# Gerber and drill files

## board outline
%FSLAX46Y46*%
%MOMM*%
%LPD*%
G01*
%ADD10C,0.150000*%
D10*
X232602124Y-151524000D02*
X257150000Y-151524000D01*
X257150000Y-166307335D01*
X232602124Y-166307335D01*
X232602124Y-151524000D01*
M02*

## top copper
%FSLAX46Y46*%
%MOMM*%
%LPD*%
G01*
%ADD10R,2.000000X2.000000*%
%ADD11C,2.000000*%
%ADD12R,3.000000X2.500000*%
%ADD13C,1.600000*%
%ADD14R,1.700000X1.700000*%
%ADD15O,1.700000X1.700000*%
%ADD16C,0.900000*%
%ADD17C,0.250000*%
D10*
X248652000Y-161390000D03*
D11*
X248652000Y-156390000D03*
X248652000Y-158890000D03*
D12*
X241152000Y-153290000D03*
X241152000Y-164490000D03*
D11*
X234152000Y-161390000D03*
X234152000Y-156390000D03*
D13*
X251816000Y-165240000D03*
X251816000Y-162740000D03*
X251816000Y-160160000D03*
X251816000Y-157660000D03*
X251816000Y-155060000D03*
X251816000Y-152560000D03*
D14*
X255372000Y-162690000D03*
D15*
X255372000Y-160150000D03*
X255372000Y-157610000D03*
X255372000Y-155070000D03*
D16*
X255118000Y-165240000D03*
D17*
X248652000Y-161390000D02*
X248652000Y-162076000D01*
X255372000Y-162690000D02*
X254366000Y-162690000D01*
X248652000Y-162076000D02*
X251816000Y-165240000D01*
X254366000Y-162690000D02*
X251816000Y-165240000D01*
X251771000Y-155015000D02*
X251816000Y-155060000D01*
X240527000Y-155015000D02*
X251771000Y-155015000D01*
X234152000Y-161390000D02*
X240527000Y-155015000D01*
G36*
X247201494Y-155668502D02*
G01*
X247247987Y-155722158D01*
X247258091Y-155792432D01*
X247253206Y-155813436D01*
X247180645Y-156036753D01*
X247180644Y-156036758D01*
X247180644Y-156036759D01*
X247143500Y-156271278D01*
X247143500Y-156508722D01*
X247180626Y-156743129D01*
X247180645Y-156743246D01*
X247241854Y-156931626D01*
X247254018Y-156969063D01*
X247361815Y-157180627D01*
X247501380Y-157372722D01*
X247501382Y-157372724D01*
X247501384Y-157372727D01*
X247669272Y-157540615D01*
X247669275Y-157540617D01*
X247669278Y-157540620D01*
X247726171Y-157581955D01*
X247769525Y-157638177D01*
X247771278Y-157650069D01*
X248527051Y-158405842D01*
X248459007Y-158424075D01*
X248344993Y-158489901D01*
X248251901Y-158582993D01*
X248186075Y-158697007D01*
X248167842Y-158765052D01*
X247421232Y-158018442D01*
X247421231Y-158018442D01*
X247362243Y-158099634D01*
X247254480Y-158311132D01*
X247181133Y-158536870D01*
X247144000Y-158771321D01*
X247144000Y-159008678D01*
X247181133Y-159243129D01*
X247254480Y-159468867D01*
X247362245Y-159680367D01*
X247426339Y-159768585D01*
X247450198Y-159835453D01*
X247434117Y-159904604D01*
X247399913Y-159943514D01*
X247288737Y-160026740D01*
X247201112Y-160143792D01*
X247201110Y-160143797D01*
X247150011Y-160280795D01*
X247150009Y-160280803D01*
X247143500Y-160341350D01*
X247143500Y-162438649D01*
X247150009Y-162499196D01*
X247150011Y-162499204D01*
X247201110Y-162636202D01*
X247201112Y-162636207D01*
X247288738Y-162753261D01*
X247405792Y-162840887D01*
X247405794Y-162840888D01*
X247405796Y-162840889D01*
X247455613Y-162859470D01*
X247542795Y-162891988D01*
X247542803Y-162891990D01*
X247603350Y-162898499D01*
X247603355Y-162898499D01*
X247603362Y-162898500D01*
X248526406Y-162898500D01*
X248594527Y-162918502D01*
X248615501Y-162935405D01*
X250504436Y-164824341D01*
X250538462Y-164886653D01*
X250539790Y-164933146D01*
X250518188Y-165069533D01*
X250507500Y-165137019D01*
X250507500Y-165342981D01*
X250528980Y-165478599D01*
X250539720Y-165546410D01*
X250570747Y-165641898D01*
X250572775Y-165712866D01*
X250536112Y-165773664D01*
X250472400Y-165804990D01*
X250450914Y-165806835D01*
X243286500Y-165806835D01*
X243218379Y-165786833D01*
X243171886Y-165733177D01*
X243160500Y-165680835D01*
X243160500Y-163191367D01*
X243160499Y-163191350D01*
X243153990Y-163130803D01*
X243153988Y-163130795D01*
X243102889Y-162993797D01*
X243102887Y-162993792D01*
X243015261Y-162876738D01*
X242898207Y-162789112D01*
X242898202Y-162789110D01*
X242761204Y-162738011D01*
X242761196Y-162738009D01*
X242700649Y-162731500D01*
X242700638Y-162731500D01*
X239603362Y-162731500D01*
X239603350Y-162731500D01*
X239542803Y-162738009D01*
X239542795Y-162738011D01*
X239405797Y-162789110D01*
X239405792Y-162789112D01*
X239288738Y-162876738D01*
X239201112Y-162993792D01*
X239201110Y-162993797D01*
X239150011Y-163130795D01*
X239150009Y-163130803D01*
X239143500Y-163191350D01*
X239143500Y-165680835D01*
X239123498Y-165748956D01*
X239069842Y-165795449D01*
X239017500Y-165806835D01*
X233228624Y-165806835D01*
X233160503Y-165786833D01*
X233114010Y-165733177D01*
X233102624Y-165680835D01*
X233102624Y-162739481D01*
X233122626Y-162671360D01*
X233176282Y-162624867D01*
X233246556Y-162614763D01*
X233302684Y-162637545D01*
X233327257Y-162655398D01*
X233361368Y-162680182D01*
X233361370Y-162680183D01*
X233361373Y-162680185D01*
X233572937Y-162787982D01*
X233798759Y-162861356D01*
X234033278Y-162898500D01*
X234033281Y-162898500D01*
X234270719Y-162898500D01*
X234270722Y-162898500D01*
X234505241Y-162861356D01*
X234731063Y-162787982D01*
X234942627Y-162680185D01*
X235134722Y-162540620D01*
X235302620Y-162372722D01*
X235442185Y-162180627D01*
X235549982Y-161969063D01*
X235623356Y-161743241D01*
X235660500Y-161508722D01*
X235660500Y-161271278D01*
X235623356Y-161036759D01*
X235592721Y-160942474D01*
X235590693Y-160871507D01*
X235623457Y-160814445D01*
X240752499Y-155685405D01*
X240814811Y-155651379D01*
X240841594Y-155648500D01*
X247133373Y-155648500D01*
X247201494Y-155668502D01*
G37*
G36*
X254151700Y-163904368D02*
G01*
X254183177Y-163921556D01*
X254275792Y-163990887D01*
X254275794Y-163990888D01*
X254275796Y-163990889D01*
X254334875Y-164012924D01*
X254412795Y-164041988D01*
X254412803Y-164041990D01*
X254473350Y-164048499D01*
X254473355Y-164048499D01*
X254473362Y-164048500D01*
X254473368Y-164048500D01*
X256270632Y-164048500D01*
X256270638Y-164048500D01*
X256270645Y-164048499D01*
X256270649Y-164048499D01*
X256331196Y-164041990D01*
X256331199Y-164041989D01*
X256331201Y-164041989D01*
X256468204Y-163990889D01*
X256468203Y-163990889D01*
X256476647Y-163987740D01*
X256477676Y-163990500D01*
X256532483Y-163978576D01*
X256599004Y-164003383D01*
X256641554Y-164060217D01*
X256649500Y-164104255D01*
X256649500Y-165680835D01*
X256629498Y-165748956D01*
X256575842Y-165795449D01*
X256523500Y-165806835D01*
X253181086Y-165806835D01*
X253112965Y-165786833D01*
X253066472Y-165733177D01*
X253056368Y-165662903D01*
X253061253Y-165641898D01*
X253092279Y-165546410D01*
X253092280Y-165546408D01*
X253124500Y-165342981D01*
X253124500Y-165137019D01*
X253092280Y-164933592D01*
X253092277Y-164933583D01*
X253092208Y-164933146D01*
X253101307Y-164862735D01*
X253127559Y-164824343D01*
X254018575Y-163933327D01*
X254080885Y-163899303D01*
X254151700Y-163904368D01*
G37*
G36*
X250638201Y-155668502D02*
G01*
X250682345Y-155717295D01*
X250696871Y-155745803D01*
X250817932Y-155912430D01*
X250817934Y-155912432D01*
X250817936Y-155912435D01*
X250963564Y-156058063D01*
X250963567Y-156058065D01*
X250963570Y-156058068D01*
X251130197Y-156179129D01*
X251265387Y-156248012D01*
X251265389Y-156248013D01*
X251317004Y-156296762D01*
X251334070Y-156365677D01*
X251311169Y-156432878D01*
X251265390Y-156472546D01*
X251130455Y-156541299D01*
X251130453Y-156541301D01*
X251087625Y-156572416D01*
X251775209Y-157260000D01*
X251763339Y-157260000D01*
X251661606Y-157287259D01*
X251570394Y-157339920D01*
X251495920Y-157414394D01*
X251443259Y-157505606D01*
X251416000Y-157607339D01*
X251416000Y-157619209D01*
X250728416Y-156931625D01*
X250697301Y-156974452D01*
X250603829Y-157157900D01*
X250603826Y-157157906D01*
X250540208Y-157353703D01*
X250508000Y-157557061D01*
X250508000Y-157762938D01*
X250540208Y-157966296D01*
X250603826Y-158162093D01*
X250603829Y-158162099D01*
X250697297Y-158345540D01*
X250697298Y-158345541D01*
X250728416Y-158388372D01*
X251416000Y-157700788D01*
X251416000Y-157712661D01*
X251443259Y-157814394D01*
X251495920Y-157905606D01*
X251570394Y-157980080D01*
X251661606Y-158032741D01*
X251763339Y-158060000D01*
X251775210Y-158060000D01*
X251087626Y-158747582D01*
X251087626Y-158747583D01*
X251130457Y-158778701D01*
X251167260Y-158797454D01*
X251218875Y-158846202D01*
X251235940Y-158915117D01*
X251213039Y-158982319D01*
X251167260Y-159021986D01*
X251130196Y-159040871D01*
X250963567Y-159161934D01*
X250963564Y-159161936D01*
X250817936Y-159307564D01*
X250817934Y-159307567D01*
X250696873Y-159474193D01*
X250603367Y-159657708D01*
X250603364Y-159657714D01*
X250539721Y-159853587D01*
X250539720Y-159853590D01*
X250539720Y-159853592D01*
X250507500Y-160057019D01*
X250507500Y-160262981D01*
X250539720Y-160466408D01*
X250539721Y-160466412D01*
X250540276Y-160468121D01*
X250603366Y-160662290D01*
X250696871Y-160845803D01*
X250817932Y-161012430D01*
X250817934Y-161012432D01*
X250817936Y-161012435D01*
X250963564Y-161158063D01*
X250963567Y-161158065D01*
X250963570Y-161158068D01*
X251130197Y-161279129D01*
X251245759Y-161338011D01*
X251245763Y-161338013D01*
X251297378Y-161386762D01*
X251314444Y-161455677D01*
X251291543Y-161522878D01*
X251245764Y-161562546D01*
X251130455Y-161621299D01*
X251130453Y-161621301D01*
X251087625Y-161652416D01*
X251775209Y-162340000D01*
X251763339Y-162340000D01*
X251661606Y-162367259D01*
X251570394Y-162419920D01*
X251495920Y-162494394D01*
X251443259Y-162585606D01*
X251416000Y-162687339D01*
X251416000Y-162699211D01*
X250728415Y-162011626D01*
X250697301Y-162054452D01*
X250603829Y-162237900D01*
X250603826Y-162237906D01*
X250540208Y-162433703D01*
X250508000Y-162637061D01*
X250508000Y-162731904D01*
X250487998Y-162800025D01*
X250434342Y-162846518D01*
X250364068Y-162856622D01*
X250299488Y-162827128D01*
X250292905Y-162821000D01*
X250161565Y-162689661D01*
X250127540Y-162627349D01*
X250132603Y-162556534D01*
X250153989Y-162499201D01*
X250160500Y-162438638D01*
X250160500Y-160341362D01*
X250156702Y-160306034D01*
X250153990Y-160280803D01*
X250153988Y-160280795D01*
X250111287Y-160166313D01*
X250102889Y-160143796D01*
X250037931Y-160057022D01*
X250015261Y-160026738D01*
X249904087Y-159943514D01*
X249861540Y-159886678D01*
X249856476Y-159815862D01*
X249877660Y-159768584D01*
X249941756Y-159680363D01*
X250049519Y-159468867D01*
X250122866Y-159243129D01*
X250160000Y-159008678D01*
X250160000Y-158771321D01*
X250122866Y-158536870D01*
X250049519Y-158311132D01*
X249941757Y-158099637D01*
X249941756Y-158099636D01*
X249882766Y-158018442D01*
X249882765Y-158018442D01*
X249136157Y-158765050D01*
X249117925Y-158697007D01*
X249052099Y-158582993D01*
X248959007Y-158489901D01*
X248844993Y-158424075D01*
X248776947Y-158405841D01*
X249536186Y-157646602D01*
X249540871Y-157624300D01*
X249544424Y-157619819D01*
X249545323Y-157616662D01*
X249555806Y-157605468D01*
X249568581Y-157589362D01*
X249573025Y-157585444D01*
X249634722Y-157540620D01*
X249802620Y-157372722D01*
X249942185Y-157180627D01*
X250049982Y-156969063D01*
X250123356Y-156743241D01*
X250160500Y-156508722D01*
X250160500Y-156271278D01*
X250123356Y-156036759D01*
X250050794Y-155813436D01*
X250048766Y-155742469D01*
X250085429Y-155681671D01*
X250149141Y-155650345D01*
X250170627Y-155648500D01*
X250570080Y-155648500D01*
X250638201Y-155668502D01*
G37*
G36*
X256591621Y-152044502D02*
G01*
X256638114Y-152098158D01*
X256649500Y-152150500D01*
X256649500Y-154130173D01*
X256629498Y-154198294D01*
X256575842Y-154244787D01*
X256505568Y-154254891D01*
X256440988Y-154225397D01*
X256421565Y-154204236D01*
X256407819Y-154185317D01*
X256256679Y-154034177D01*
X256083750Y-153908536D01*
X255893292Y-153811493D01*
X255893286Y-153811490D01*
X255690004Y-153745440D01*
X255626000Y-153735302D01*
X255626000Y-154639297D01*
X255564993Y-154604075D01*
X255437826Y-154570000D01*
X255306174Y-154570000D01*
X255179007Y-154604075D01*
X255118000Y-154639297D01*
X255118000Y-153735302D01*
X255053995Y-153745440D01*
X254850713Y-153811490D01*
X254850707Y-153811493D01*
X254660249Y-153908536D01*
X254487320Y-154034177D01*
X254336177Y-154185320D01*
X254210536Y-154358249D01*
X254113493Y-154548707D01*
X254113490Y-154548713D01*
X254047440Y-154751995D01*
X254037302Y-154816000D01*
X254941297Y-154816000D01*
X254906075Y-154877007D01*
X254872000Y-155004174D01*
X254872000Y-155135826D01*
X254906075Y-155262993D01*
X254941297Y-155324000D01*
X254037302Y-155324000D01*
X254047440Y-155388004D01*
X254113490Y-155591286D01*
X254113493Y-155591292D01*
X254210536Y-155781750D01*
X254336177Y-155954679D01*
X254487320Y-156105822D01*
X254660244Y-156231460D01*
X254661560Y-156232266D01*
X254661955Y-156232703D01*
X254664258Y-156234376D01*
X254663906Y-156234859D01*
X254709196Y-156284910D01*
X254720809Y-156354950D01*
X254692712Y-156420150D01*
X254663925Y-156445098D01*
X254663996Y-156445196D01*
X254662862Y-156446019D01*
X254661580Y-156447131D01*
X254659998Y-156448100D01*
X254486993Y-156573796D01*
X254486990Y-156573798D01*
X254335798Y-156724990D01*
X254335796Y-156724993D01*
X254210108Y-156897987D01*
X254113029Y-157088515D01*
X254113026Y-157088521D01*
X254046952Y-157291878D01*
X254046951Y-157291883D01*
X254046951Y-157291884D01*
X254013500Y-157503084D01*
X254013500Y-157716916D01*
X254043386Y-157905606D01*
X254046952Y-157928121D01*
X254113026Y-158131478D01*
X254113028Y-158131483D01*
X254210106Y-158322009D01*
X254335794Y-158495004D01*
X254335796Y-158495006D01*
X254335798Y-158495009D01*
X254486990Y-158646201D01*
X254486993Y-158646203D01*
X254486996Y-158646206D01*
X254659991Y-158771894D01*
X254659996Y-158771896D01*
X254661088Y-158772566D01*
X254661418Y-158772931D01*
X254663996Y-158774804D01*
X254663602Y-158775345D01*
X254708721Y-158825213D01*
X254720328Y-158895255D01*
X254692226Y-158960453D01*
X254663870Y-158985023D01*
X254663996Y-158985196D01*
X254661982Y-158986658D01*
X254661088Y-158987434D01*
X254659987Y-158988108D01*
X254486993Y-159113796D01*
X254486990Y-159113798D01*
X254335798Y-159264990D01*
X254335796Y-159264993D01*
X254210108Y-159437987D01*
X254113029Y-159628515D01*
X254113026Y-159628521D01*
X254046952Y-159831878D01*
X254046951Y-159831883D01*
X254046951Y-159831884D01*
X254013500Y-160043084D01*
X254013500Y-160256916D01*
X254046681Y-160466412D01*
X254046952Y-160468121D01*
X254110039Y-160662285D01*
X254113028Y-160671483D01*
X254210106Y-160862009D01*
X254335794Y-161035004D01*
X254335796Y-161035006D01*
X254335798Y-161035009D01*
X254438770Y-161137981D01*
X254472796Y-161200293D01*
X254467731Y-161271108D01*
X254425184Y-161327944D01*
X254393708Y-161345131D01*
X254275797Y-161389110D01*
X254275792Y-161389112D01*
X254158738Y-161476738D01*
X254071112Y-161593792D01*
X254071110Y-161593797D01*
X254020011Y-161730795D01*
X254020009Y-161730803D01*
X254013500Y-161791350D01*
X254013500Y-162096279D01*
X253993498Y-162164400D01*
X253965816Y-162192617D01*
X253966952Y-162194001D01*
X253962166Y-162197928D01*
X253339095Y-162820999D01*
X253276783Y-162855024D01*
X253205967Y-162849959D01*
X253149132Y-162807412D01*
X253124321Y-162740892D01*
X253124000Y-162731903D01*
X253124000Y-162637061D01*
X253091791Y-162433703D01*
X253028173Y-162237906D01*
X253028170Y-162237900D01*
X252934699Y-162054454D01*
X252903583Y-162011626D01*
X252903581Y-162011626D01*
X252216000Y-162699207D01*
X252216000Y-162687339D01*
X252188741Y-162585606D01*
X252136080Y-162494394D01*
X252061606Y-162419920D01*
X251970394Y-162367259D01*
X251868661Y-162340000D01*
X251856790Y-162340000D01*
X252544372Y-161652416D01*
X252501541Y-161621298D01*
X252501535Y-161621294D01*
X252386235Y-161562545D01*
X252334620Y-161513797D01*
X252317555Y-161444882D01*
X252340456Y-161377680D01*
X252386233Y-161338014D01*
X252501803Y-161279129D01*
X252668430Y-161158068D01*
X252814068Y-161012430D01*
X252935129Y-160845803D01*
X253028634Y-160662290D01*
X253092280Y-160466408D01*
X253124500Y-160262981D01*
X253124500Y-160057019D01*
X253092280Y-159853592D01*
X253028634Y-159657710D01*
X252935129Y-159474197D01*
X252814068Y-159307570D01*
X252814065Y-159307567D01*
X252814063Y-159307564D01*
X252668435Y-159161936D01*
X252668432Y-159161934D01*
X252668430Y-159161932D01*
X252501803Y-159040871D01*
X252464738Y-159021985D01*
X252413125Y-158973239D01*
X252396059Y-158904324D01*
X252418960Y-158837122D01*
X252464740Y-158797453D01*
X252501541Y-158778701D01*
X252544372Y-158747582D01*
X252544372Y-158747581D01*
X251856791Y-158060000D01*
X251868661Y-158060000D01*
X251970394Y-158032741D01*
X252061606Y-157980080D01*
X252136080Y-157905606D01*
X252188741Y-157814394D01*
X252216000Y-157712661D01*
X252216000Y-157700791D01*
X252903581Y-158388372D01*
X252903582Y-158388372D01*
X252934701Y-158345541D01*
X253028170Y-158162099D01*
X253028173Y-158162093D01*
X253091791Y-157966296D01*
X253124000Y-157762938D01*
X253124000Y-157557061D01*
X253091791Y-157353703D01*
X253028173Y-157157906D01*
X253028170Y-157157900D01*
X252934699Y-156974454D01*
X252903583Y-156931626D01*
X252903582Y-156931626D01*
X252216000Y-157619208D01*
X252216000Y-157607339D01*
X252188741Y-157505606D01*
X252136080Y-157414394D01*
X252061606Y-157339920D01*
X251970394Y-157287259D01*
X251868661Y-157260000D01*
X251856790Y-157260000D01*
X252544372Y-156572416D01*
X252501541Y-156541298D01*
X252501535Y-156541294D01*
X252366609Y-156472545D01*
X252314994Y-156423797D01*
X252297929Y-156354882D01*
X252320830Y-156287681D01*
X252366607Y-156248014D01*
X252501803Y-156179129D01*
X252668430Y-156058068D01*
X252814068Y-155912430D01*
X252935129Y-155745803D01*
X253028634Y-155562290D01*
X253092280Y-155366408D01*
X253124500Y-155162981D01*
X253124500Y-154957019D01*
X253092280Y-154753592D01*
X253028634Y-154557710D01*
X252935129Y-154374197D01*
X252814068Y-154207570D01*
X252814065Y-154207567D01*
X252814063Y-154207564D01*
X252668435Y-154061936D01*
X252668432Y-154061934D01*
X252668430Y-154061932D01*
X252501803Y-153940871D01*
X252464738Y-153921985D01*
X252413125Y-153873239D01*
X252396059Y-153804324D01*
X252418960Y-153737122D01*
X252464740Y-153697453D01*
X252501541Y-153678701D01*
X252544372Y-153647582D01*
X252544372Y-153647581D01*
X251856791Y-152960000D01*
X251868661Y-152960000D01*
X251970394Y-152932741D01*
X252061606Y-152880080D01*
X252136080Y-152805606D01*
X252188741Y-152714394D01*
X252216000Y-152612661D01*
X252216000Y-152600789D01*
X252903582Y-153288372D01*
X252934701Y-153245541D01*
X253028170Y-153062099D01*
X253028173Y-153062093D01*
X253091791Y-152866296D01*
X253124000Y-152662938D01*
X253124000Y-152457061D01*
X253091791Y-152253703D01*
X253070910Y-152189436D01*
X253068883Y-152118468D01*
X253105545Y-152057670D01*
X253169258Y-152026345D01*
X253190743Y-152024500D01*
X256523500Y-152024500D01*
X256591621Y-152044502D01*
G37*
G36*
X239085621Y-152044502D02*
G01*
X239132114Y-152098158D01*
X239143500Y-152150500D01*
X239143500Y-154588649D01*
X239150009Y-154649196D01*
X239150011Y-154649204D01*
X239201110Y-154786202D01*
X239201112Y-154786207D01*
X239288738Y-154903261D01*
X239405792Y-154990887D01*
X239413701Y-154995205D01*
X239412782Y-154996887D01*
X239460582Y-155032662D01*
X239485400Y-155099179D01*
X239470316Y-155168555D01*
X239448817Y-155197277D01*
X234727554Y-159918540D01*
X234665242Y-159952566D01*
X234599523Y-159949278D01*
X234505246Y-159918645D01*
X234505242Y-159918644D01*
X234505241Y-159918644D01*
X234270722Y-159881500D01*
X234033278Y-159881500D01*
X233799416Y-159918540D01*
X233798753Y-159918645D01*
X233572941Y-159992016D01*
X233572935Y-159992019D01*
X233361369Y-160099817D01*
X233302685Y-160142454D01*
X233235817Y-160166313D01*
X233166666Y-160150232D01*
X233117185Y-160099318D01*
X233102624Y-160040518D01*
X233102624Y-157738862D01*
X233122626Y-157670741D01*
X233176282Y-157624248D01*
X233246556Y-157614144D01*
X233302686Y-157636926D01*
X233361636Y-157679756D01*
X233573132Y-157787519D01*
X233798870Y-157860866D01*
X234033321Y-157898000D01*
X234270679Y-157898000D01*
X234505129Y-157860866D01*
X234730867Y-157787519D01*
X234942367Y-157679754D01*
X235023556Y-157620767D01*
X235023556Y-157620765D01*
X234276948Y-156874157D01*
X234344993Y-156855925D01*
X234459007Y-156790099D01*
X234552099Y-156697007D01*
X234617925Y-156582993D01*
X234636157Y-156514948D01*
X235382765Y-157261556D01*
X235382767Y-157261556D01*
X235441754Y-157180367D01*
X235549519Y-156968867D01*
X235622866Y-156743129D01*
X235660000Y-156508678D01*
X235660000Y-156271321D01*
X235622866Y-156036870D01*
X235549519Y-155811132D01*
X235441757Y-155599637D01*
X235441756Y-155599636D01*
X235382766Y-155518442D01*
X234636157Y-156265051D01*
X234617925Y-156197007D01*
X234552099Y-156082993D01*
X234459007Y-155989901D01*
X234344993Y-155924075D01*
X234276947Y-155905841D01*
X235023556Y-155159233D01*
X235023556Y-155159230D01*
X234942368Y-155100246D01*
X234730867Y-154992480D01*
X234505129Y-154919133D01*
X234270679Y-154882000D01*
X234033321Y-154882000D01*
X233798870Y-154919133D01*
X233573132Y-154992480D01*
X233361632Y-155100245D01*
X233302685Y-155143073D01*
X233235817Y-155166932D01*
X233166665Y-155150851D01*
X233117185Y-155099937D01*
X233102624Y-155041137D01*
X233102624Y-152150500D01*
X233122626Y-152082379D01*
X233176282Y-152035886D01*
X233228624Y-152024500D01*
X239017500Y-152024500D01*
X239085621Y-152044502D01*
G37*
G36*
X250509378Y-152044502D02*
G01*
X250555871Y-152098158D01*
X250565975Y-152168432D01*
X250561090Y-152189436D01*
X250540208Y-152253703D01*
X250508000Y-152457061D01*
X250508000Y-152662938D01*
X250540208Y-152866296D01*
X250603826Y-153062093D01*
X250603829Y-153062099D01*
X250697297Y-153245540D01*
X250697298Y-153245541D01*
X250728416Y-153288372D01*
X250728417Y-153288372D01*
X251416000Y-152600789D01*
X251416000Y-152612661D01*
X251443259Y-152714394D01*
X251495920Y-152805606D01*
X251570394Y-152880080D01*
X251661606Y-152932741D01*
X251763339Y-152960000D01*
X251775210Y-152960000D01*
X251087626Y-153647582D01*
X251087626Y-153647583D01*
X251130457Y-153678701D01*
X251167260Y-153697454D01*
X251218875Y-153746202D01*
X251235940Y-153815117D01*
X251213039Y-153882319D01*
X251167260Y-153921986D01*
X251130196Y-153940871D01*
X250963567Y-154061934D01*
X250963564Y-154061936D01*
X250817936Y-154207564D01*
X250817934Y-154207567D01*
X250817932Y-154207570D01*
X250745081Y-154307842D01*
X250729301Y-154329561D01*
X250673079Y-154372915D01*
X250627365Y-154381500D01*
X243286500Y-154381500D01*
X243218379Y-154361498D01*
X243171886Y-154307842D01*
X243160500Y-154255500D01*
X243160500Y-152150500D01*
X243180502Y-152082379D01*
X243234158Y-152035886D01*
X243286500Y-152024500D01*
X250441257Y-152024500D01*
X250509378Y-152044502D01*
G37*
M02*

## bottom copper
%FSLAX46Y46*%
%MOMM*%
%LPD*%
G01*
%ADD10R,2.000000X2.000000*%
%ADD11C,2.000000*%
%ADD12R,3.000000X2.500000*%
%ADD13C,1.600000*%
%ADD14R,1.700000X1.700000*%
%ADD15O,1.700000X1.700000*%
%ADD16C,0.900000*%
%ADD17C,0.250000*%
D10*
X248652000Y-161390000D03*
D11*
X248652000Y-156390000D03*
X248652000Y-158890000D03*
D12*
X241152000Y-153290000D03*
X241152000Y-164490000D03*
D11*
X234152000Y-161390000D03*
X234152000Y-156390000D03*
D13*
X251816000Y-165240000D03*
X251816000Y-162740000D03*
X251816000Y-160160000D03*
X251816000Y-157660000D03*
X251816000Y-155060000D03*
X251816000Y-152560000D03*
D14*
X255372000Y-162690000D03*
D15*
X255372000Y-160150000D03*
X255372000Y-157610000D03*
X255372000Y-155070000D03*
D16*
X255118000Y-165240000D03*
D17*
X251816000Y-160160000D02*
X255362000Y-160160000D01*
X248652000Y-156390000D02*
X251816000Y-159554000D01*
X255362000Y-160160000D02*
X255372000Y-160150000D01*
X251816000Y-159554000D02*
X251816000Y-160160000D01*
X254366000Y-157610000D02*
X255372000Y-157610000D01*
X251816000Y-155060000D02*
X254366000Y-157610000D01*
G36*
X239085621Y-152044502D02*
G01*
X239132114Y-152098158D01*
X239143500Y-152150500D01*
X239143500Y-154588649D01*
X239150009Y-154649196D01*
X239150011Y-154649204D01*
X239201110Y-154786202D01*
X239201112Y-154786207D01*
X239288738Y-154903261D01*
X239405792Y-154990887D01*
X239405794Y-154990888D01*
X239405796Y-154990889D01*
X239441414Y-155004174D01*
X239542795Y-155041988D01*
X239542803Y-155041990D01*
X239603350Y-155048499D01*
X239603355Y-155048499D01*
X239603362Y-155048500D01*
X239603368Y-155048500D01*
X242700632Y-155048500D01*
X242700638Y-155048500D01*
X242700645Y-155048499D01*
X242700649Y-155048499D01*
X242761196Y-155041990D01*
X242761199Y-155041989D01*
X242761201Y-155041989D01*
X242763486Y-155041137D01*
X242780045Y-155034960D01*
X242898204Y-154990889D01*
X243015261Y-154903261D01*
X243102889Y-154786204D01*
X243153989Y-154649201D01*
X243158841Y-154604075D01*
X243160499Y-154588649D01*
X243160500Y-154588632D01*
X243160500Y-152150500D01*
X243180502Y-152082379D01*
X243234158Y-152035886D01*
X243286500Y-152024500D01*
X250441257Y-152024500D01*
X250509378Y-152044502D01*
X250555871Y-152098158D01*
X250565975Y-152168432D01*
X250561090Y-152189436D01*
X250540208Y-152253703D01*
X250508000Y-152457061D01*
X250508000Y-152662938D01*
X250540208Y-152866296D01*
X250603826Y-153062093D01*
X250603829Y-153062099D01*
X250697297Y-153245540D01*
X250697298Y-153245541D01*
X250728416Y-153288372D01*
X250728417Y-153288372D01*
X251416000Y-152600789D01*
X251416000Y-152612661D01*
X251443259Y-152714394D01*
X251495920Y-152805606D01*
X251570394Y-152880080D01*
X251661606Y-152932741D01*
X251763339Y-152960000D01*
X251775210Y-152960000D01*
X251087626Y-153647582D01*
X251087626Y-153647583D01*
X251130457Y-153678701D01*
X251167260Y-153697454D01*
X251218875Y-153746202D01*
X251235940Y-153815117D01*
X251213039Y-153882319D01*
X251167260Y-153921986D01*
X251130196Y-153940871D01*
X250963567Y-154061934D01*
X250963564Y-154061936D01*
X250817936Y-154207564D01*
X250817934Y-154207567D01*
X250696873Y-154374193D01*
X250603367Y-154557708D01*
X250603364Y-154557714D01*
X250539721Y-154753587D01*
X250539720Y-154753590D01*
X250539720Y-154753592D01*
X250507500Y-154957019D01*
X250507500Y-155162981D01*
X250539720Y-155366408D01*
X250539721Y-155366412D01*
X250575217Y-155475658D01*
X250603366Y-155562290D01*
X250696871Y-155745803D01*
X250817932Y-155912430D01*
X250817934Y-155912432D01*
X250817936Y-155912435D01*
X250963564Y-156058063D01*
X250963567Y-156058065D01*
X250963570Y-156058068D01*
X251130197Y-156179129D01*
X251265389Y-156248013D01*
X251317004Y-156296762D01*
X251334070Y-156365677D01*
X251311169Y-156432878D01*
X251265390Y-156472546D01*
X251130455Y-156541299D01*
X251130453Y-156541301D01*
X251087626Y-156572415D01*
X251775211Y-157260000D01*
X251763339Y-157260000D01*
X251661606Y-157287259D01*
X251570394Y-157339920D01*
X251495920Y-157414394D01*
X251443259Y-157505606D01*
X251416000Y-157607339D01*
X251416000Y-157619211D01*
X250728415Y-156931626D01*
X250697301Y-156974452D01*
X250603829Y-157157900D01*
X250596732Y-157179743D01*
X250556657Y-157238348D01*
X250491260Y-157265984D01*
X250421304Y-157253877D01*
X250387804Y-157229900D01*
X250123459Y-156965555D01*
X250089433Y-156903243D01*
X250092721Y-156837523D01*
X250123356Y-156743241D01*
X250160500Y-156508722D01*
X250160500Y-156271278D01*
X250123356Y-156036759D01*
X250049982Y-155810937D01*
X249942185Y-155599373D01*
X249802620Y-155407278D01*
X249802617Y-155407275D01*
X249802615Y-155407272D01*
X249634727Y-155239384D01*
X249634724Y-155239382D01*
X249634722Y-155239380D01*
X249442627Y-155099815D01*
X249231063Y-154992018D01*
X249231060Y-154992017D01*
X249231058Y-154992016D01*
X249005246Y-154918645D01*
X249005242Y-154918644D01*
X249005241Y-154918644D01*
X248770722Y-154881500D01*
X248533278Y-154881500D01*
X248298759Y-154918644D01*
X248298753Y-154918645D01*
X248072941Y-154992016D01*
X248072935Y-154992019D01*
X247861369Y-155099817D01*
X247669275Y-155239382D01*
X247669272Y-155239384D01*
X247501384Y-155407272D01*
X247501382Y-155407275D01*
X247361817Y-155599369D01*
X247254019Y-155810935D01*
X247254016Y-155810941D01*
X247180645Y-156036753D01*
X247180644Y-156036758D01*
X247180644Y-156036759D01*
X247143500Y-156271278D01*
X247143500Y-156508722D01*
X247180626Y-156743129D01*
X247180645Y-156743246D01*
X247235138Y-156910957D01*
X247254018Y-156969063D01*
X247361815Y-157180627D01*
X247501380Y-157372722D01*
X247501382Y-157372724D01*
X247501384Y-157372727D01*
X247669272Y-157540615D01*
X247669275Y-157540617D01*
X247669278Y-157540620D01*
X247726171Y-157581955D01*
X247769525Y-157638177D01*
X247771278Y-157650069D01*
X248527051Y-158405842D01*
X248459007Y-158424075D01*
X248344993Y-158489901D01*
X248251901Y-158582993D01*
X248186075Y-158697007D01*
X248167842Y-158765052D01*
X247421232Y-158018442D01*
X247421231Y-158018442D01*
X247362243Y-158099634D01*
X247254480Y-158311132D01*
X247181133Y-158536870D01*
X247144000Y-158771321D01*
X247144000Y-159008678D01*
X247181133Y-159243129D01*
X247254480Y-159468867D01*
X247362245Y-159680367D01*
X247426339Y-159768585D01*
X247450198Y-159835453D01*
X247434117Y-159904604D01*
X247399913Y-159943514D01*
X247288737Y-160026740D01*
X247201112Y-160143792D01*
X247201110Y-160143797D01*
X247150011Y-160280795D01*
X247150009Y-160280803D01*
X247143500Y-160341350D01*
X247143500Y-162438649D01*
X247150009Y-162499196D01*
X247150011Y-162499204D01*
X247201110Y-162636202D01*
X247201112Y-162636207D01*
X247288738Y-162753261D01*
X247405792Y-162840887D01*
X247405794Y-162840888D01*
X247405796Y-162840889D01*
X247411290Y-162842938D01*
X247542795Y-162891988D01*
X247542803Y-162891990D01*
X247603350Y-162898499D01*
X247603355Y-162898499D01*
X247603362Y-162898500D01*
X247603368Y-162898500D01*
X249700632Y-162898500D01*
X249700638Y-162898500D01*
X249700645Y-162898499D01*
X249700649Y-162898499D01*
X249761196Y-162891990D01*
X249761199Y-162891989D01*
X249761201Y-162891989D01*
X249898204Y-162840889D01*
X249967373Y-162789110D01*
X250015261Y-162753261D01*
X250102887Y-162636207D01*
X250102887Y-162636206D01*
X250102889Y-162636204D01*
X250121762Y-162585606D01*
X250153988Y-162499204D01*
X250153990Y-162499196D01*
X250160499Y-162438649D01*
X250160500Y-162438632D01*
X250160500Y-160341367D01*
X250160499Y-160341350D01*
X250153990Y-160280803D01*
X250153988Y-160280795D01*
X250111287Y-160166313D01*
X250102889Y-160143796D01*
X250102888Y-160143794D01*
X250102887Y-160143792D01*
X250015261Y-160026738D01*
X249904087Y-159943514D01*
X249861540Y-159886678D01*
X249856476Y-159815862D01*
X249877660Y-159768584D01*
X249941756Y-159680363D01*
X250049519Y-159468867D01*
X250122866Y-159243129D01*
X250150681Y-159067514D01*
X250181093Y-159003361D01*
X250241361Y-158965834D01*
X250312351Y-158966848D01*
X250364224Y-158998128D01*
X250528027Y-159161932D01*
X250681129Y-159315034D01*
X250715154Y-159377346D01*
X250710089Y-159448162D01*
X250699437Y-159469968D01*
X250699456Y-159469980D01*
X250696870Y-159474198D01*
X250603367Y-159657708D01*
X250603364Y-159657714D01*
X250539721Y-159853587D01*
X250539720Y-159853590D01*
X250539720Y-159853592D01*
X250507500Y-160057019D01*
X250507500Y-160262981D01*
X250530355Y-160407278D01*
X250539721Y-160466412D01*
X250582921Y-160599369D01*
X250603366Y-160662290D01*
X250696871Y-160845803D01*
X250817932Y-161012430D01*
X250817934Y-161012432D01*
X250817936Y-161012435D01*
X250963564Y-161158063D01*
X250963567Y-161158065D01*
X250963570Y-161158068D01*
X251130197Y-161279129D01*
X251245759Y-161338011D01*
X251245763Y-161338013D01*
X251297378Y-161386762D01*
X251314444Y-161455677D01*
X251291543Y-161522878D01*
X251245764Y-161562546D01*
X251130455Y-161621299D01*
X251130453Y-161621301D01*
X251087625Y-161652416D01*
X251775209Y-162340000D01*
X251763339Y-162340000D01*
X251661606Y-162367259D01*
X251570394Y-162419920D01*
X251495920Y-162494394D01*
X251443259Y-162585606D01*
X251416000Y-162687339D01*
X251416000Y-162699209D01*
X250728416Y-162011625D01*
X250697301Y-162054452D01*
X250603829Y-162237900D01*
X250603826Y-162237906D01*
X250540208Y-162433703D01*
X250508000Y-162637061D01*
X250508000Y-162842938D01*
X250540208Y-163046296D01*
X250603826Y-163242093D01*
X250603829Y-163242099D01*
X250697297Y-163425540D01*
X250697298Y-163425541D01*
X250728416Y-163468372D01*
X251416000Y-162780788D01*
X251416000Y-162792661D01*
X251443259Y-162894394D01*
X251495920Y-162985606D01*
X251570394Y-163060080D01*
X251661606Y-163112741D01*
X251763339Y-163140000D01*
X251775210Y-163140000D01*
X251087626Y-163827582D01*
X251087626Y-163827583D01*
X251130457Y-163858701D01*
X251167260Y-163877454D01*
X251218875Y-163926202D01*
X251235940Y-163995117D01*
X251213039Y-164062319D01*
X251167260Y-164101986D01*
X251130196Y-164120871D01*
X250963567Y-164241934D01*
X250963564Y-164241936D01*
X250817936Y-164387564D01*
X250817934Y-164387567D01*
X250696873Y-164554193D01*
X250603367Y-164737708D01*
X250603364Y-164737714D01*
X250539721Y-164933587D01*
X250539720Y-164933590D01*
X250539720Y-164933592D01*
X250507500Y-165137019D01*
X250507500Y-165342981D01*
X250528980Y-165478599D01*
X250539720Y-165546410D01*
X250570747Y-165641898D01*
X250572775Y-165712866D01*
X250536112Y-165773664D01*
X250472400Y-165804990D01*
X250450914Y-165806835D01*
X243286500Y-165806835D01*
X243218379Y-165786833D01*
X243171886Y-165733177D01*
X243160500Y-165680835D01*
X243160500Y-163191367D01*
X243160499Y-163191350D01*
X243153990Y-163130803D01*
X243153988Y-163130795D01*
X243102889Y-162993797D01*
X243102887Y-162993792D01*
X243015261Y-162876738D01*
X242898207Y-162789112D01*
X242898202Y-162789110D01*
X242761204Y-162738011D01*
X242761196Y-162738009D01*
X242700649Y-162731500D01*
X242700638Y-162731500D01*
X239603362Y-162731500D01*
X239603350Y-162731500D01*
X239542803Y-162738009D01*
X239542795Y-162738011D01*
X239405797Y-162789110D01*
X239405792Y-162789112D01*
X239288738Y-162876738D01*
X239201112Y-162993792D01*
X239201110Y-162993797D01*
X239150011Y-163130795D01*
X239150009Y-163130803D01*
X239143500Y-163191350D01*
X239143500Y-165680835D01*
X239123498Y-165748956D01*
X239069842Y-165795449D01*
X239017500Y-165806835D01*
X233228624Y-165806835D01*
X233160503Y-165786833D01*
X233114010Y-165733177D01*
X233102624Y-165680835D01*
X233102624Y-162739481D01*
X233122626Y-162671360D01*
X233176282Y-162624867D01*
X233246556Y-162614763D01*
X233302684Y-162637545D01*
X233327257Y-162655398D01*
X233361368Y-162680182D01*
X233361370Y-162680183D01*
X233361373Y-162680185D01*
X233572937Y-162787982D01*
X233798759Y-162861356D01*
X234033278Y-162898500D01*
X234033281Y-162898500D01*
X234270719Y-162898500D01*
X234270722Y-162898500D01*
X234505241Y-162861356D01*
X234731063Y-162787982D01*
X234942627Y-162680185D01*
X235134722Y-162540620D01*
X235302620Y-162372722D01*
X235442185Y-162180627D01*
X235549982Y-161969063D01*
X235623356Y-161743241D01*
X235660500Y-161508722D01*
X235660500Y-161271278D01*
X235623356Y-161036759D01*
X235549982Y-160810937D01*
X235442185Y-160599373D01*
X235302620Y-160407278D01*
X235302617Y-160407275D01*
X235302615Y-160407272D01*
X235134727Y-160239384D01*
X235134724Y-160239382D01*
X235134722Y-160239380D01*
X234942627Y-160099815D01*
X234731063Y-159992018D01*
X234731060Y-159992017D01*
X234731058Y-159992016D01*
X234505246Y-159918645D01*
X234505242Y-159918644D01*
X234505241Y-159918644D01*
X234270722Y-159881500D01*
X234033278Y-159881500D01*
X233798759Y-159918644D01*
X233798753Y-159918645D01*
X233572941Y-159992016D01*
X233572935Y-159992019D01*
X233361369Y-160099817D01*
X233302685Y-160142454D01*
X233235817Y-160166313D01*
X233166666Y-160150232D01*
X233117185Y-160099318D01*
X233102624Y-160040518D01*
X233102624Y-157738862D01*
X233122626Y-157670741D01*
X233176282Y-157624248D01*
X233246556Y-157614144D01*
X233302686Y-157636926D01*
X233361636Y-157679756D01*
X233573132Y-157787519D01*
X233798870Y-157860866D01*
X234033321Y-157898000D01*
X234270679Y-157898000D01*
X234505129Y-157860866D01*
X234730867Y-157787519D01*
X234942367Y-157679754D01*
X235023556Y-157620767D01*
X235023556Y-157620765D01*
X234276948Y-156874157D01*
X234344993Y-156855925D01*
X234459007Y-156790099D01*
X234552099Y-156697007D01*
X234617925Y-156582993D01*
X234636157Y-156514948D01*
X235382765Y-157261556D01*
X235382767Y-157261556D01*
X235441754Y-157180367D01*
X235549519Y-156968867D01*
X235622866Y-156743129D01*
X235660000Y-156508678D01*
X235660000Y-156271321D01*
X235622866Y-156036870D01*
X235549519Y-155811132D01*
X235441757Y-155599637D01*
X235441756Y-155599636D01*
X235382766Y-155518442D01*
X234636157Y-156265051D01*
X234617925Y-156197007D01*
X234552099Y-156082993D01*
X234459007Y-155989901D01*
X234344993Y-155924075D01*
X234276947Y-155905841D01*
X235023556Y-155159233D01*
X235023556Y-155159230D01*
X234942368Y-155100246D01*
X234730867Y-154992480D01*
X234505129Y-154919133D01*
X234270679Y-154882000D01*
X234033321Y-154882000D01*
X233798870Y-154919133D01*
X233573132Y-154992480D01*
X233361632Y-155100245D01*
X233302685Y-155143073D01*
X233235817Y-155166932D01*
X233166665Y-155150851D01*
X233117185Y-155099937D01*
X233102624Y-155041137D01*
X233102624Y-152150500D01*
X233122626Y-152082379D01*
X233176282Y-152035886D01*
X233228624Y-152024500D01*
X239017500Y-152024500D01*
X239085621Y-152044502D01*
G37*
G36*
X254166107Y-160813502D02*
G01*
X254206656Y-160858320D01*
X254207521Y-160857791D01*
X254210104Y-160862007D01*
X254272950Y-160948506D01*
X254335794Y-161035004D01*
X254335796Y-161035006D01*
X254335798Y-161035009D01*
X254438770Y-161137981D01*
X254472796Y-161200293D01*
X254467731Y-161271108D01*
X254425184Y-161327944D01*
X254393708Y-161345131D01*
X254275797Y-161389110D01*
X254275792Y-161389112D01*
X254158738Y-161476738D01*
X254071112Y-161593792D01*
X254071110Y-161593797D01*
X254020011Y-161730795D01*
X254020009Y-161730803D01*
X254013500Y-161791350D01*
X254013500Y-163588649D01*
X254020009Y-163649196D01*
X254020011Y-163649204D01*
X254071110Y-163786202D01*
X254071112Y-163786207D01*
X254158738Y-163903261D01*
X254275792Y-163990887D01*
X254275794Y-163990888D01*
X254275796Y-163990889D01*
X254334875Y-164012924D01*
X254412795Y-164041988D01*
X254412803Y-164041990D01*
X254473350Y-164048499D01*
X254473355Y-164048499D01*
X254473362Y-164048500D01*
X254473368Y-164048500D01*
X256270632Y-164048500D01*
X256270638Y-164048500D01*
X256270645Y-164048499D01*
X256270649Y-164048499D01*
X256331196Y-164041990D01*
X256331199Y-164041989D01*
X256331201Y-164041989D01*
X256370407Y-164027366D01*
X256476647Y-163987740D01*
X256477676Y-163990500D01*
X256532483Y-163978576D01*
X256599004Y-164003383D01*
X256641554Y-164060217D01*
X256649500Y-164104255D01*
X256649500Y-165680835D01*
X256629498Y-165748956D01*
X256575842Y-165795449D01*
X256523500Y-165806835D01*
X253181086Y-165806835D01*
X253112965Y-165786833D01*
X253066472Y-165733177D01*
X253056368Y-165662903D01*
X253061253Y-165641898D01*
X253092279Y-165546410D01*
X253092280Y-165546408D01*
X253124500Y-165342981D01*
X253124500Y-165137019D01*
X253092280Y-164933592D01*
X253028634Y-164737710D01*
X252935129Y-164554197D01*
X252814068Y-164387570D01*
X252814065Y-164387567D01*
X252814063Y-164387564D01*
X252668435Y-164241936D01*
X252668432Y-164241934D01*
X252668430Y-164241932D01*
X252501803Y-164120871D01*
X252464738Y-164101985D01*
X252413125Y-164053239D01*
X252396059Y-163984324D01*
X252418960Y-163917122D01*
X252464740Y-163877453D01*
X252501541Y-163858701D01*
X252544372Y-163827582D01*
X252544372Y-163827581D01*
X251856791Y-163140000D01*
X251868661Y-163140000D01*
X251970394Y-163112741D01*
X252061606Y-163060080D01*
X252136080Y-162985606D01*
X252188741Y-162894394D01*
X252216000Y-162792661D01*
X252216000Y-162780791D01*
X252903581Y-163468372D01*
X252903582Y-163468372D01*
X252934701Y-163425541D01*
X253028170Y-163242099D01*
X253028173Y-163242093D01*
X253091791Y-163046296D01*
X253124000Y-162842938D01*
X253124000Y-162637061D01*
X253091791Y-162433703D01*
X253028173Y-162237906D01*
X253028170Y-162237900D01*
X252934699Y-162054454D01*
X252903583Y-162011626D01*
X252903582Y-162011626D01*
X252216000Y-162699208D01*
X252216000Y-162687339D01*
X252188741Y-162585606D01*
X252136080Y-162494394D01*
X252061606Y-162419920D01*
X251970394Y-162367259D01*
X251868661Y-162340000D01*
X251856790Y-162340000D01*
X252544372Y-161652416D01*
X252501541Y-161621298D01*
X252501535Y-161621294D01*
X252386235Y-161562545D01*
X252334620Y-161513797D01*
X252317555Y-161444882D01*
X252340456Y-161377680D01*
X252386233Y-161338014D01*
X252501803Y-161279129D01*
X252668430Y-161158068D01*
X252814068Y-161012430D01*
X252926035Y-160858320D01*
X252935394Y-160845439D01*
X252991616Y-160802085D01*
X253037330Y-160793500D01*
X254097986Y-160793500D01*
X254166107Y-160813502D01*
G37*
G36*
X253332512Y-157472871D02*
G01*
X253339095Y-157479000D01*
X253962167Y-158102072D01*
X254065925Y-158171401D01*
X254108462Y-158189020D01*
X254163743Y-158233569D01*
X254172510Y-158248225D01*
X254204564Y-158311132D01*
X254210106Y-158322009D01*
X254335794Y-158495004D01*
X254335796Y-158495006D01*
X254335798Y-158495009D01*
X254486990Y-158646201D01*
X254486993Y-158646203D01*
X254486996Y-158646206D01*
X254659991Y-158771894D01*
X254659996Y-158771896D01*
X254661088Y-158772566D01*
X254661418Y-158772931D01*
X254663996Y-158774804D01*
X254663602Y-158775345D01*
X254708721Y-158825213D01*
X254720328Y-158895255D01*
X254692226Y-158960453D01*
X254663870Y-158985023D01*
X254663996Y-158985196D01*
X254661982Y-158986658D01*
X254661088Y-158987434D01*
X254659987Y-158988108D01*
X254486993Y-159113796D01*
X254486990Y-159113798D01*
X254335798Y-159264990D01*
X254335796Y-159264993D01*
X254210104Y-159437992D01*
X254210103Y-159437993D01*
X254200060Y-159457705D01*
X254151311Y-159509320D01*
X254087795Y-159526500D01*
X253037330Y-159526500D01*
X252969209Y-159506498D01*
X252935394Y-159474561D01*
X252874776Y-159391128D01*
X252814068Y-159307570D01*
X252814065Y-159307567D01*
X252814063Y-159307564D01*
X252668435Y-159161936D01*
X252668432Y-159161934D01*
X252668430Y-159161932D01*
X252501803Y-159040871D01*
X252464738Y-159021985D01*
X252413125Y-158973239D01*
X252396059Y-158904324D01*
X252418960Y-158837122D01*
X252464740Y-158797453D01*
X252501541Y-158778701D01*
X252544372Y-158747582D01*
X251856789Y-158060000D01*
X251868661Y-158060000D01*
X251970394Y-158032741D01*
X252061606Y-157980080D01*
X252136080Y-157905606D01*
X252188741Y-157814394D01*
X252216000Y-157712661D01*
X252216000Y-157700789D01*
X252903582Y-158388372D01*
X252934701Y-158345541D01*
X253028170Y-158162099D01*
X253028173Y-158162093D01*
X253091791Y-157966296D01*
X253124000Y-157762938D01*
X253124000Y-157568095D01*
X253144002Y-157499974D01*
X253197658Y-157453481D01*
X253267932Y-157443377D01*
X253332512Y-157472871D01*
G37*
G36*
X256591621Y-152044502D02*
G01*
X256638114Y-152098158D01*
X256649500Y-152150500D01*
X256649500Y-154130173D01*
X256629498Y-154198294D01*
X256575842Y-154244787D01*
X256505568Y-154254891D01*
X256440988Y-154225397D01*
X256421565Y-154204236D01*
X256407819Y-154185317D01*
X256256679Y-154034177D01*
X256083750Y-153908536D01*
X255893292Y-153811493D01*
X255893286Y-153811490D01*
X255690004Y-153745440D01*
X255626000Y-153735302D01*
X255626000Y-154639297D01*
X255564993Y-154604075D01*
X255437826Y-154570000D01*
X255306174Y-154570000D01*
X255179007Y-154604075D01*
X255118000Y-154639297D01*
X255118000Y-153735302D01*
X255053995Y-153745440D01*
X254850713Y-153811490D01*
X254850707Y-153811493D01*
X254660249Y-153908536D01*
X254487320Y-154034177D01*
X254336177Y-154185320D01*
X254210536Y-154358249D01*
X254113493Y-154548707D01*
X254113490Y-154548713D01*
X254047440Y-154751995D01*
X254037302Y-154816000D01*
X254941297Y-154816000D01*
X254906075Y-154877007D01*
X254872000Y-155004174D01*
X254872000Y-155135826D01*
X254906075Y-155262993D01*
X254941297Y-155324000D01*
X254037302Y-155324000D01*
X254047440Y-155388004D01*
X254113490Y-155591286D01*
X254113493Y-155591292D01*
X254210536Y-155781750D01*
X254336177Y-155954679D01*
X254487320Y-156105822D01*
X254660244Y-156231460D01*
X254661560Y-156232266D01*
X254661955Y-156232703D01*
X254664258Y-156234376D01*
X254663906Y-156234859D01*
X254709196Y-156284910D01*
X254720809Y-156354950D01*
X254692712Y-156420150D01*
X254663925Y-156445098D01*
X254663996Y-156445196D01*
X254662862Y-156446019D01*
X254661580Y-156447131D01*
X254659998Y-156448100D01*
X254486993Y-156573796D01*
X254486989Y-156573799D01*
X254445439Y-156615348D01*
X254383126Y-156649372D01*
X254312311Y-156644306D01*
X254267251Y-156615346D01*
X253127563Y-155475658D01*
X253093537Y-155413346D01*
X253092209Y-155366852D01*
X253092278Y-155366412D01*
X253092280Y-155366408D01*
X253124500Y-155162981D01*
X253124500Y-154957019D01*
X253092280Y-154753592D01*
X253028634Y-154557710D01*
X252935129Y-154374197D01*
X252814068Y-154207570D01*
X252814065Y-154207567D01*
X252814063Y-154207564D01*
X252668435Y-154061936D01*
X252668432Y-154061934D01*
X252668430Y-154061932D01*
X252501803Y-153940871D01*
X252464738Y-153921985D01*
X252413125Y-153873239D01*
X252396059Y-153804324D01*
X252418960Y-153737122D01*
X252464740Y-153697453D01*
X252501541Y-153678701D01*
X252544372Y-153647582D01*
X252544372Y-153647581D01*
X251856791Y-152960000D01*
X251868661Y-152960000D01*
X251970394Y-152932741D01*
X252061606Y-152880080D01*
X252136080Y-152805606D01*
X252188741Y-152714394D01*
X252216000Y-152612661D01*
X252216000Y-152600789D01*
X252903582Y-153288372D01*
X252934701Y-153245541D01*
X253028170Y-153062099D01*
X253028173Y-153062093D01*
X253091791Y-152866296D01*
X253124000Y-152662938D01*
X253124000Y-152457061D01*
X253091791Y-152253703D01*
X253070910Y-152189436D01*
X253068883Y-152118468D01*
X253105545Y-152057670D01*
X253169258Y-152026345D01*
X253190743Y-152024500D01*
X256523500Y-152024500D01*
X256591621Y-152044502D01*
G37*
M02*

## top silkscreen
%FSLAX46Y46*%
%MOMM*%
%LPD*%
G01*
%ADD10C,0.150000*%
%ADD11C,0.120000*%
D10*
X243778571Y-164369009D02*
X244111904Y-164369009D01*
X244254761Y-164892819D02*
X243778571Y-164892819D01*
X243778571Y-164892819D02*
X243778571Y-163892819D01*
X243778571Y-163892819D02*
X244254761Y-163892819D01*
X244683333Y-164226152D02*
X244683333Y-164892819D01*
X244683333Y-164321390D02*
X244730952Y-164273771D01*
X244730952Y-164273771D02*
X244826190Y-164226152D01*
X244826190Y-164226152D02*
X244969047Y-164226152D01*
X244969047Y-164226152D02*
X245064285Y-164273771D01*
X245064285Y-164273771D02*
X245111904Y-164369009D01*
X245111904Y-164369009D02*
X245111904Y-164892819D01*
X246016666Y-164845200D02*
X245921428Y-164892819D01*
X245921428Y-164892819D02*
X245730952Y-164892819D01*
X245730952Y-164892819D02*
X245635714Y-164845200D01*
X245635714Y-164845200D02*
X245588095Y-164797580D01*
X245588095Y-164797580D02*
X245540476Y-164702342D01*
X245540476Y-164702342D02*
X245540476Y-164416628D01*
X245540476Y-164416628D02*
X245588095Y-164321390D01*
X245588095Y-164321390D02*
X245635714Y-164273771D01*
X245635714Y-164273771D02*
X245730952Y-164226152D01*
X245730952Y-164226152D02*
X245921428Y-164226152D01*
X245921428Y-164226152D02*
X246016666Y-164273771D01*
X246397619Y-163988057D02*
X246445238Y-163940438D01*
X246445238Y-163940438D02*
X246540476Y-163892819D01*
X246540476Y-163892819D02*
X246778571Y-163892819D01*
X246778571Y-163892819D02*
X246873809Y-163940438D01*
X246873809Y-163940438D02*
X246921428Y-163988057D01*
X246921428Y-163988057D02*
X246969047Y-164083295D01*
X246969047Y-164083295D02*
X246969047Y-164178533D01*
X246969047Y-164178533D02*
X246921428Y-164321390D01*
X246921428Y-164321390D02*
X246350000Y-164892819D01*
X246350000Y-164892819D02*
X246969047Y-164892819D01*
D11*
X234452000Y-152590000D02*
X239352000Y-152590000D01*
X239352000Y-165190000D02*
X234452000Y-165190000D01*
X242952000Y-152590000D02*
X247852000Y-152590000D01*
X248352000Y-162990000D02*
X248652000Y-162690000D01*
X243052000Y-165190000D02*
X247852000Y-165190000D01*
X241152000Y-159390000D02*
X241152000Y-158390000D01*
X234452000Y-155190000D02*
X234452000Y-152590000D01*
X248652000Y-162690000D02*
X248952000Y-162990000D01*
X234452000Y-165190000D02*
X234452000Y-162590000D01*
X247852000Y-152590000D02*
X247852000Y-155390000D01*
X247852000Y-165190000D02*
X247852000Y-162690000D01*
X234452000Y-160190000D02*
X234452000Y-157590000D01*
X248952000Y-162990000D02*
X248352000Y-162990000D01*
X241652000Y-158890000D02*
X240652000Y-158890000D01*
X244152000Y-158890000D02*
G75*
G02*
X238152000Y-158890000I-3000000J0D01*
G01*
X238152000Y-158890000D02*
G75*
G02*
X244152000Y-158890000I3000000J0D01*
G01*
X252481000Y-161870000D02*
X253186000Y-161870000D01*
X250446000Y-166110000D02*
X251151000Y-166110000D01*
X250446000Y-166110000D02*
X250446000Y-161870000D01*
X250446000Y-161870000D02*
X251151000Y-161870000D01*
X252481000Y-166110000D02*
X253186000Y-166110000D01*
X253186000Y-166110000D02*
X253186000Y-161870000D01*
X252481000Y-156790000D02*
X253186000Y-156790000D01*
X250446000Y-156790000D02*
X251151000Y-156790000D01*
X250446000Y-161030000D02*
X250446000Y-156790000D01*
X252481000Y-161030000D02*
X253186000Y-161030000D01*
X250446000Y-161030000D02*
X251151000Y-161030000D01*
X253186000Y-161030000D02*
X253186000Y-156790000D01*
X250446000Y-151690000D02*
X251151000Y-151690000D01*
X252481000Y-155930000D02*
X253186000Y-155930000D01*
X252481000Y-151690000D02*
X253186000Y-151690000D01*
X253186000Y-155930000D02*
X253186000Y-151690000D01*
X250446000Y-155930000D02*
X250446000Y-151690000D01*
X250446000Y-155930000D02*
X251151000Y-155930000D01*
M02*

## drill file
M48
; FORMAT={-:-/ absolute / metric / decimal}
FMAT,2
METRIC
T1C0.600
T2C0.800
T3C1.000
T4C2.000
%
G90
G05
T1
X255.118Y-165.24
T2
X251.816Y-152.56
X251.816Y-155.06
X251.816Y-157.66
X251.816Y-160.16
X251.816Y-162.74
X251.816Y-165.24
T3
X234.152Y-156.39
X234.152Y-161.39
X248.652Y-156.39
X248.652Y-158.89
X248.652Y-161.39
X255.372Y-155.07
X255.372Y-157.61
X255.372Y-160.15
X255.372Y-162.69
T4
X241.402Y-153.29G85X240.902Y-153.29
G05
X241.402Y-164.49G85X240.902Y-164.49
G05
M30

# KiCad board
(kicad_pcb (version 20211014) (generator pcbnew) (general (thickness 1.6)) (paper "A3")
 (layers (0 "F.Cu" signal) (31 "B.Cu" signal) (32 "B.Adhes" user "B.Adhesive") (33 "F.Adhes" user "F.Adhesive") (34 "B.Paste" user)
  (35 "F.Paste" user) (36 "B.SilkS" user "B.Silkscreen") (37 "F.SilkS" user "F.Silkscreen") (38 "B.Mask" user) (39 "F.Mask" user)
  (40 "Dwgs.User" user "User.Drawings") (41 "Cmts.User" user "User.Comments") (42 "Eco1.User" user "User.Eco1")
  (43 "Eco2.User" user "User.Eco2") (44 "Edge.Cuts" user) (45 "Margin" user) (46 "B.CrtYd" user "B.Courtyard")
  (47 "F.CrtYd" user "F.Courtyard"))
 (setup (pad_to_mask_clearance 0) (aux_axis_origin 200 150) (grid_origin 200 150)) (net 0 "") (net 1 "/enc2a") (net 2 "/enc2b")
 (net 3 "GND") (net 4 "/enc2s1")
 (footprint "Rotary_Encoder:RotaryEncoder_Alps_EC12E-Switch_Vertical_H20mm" (layer "F.Cu") (at 248.652 161.39 180)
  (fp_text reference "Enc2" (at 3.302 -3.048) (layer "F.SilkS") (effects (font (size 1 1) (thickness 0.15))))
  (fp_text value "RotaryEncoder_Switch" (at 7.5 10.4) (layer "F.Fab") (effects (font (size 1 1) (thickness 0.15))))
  (fp_line (start 14.2 8.8) (end 9.3 8.8) (layer "F.SilkS") (width 0.12))
  (fp_line (start 9.3 -3.8) (end 14.2 -3.8) (layer "F.SilkS") (width 0.12))
  (fp_line (start 5.7 8.8) (end 0.8 8.8) (layer "F.SilkS") (width 0.12))
  (fp_line (start 0.3 -1.6) (end 0 -1.3) (layer "F.SilkS") (width 0.12))
  (fp_line (start 5.6 -3.8) (end 0.8 -3.8) (layer "F.SilkS") (width 0.12))
  (fp_line (start 7.5 2) (end 7.5 3) (layer "F.SilkS") (width 0.12))
  (fp_line (start 14.2 6.2) (end 14.2 8.8) (layer "F.SilkS") (width 0.12))
  (fp_line (start 0 -1.3) (end -0.3 -1.6) (layer "F.SilkS") (width 0.12))
  (fp_line (start 14.2 -3.8) (end 14.2 -1.2) (layer "F.SilkS") (width 0.12))
  (fp_line (start 0.8 8.8) (end 0.8 6) (layer "F.SilkS") (width 0.12))
  (fp_line (start 0.8 -3.8) (end 0.8 -1.3) (layer "F.SilkS") (width 0.12))
  (fp_line (start 14.2 1.2) (end 14.2 3.8) (layer "F.SilkS") (width 0.12))
  (fp_line (start -0.3 -1.6) (end 0.3 -1.6) (layer "F.SilkS") (width 0.12))
  (fp_line (start 7 2.5) (end 8 2.5) (layer "F.SilkS") (width 0.12))
  (fp_circle (center 7.5 2.5) (end 10.5 2.5) (layer "F.SilkS") (width 0.12) (fill none))
  (pad "A" thru_hole rect (at 0 0 180) (size 2 2) (drill 1) (layers *.Cu *.Mask) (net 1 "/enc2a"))
  (pad "B" thru_hole circle (at 0 5 180) (size 2 2) (drill 1) (layers *.Cu *.Mask) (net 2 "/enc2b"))
  (pad "C" thru_hole circle (at 0 2.5 180) (size 2 2) (drill 1) (layers *.Cu *.Mask) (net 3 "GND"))
  (pad "MP" thru_hole rect (at 7.5 8.1 180) (size 3 2.5) (drill oval 2.5 2) (layers *.Cu *.Mask))
  (pad "MP" thru_hole rect (at 7.5 -3.1 180) (size 3 2.5) (drill oval 2.5 2) (layers *.Cu *.Mask))
  (pad "S1" thru_hole circle (at 14.5 0 180) (size 2 2) (drill 1) (layers *.Cu *.Mask) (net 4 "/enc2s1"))
  (pad "S2" thru_hole circle (at 14.5 5 180) (size 2 2) (drill 1) (layers *.Cu *.Mask) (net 3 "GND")))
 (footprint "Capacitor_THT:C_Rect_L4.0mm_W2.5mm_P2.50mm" (layer "F.Cu") (at 251.816 165.24 90)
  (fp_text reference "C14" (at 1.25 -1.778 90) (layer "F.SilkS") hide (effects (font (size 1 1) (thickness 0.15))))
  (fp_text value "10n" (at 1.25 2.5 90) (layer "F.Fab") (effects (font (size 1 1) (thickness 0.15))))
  (fp_line (start 3.37 0.665) (end 3.37 1.37) (layer "F.SilkS") (width 0.12))
  (fp_line (start -0.87 -1.37) (end -0.87 -0.665) (layer "F.SilkS") (width 0.12))
  (fp_line (start -0.87 -1.37) (end 3.37 -1.37) (layer "F.SilkS") (width 0.12))
  (fp_line (start 3.37 -1.37) (end 3.37 -0.665) (layer "F.SilkS") (width 0.12))
  (fp_line (start -0.87 0.665) (end -0.87 1.37) (layer "F.SilkS") (width 0.12))
  (fp_line (start -0.87 1.37) (end 3.37 1.37) (layer "F.SilkS") (width 0.12))
  (pad "1" thru_hole circle (at 0 0 90) (size 1.6 1.6) (drill 0.8) (layers *.Cu *.Mask) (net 1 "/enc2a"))
  (pad "2" thru_hole circle (at 2.5 0 90) (size 1.6 1.6) (drill 0.8) (layers *.Cu *.Mask) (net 3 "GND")))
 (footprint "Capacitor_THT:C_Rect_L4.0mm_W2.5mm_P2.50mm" (layer "F.Cu") (at 251.816 160.16 90)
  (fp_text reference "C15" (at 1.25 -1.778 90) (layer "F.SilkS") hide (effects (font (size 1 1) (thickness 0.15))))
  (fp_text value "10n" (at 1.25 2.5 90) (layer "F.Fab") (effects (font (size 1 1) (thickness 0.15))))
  (fp_line (start 3.37 0.665) (end 3.37 1.37) (layer "F.SilkS") (width 0.12))
  (fp_line (start 3.37 -1.37) (end 3.37 -0.665) (layer "F.SilkS") (width 0.12))
  (fp_line (start -0.87 -1.37) (end 3.37 -1.37) (layer "F.SilkS") (width 0.12))
  (fp_line (start -0.87 0.665) (end -0.87 1.37) (layer "F.SilkS") (width 0.12))
  (fp_line (start -0.87 -1.37) (end -0.87 -0.665) (layer "F.SilkS") (width 0.12))
  (fp_line (start -0.87 1.37) (end 3.37 1.37) (layer "F.SilkS") (width 0.12))
  (pad "1" thru_hole circle (at 0 0 90) (size 1.6 1.6) (drill 0.8) (layers *.Cu *.Mask) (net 2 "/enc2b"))
  (pad "2" thru_hole circle (at 2.5 0 90) (size 1.6 1.6) (drill 0.8) (layers *.Cu *.Mask) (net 3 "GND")))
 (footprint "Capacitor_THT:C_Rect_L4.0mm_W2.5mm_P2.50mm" (layer "F.Cu") (at 251.816 155.06 90)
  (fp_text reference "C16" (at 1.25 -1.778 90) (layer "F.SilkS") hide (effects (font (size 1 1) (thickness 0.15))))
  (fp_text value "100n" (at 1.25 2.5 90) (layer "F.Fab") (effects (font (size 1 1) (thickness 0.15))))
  (fp_line (start 3.37 -1.37) (end 3.37 -0.665) (layer "F.SilkS") (width 0.12))
  (fp_line (start -0.87 0.665) (end -0.87 1.37) (layer "F.SilkS") (width 0.12))
  (fp_line (start 3.37 0.665) (end 3.37 1.37) (layer "F.SilkS") (width 0.12))
  (fp_line (start -0.87 1.37) (end 3.37 1.37) (layer "F.SilkS") (width 0.12))
  (fp_line (start -0.87 -1.37) (end 3.37 -1.37) (layer "F.SilkS") (width 0.12))
  (fp_line (start -0.87 -1.37) (end -0.87 -0.665) (layer "F.SilkS") (width 0.12))
  (pad "1" thru_hole circle (at 0 0 90) (size 1.6 1.6) (drill 0.8) (layers *.Cu *.Mask) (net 4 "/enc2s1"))
  (pad "2" thru_hole circle (at 2.5 0 90) (size 1.6 1.6) (drill 0.8) (layers *.Cu *.Mask) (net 3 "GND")))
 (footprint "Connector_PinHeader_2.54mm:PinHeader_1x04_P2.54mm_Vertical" (layer "B.Cu") (at 255.372 162.69)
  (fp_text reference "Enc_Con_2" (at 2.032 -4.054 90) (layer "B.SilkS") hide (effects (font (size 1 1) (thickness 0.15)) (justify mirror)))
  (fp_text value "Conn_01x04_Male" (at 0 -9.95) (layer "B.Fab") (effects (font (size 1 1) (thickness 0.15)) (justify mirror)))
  (pad "1" thru_hole rect (at 0 0) (size 1.7 1.7) (drill 1) (layers *.Cu *.Mask) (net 1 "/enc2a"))
  (pad "2" thru_hole oval (at 0 -2.54) (size 1.7 1.7) (drill 1) (layers *.Cu *.Mask) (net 2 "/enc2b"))
  (pad "3" thru_hole oval (at 0 -5.08) (size 1.7 1.7) (drill 1) (layers *.Cu *.Mask) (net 4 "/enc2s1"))
  (pad "4" thru_hole oval (at 0 -7.62) (size 1.7 1.7) (drill 1) (layers *.Cu *.Mask) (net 3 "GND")))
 (gr_rect (start 232.602124 151.524) (end 257.15 166.307335) (layer "Edge.Cuts") (width 0.15) (fill none))
 (via (at 255.118 165.24) (size 0.9) (drill 0.6) (layers "F.Cu" "B.Cu") (free) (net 3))
 (segment (start 248.652 161.39) (end 248.652 162.076) (width 0.25) (layer "F.Cu") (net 1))
 (segment (start 255.372 162.69) (end 254.366 162.69) (width 0.25) (layer "F.Cu") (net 1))
 (segment (start 248.652 162.076) (end 251.816 165.24) (width 0.25) (layer "F.Cu") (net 1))
 (segment (start 254.366 162.69) (end 251.816 165.24) (width 0.25) (layer "F.Cu") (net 1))
 (segment (start 251.816 160.16) (end 255.362 160.16) (width 0.25) (layer "B.Cu") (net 2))
 (segment (start 248.652 156.39) (end 251.816 159.554) (width 0.25) (layer "B.Cu") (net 2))
 (segment (start 255.362 160.16) (end 255.372 160.15) (width 0.25) (layer "B.Cu") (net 2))
 (segment (start 251.816 159.554) (end 251.816 160.16) (width 0.25) (layer "B.Cu") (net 2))
 (segment (start 251.771 155.015) (end 251.816 155.06) (width 0.25) (layer "F.Cu") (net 4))
 (segment (start 240.527 155.015) (end 251.771 155.015) (width 0.25) (layer "F.Cu") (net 4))
 (segment (start 234.152 161.39) (end 240.527 155.015) (width 0.25) (layer "F.Cu") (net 4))
 (segment (start 254.366 157.61) (end 255.372 157.61) (width 0.25) (layer "B.Cu") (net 4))
 (segment (start 251.816 155.06) (end 254.366 157.61) (width 0.25) (layer "B.Cu") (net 4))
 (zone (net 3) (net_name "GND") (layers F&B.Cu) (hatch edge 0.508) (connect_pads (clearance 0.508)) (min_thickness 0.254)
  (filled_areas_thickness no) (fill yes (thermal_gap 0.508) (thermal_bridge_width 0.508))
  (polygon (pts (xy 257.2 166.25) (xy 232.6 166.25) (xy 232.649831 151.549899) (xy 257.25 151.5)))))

